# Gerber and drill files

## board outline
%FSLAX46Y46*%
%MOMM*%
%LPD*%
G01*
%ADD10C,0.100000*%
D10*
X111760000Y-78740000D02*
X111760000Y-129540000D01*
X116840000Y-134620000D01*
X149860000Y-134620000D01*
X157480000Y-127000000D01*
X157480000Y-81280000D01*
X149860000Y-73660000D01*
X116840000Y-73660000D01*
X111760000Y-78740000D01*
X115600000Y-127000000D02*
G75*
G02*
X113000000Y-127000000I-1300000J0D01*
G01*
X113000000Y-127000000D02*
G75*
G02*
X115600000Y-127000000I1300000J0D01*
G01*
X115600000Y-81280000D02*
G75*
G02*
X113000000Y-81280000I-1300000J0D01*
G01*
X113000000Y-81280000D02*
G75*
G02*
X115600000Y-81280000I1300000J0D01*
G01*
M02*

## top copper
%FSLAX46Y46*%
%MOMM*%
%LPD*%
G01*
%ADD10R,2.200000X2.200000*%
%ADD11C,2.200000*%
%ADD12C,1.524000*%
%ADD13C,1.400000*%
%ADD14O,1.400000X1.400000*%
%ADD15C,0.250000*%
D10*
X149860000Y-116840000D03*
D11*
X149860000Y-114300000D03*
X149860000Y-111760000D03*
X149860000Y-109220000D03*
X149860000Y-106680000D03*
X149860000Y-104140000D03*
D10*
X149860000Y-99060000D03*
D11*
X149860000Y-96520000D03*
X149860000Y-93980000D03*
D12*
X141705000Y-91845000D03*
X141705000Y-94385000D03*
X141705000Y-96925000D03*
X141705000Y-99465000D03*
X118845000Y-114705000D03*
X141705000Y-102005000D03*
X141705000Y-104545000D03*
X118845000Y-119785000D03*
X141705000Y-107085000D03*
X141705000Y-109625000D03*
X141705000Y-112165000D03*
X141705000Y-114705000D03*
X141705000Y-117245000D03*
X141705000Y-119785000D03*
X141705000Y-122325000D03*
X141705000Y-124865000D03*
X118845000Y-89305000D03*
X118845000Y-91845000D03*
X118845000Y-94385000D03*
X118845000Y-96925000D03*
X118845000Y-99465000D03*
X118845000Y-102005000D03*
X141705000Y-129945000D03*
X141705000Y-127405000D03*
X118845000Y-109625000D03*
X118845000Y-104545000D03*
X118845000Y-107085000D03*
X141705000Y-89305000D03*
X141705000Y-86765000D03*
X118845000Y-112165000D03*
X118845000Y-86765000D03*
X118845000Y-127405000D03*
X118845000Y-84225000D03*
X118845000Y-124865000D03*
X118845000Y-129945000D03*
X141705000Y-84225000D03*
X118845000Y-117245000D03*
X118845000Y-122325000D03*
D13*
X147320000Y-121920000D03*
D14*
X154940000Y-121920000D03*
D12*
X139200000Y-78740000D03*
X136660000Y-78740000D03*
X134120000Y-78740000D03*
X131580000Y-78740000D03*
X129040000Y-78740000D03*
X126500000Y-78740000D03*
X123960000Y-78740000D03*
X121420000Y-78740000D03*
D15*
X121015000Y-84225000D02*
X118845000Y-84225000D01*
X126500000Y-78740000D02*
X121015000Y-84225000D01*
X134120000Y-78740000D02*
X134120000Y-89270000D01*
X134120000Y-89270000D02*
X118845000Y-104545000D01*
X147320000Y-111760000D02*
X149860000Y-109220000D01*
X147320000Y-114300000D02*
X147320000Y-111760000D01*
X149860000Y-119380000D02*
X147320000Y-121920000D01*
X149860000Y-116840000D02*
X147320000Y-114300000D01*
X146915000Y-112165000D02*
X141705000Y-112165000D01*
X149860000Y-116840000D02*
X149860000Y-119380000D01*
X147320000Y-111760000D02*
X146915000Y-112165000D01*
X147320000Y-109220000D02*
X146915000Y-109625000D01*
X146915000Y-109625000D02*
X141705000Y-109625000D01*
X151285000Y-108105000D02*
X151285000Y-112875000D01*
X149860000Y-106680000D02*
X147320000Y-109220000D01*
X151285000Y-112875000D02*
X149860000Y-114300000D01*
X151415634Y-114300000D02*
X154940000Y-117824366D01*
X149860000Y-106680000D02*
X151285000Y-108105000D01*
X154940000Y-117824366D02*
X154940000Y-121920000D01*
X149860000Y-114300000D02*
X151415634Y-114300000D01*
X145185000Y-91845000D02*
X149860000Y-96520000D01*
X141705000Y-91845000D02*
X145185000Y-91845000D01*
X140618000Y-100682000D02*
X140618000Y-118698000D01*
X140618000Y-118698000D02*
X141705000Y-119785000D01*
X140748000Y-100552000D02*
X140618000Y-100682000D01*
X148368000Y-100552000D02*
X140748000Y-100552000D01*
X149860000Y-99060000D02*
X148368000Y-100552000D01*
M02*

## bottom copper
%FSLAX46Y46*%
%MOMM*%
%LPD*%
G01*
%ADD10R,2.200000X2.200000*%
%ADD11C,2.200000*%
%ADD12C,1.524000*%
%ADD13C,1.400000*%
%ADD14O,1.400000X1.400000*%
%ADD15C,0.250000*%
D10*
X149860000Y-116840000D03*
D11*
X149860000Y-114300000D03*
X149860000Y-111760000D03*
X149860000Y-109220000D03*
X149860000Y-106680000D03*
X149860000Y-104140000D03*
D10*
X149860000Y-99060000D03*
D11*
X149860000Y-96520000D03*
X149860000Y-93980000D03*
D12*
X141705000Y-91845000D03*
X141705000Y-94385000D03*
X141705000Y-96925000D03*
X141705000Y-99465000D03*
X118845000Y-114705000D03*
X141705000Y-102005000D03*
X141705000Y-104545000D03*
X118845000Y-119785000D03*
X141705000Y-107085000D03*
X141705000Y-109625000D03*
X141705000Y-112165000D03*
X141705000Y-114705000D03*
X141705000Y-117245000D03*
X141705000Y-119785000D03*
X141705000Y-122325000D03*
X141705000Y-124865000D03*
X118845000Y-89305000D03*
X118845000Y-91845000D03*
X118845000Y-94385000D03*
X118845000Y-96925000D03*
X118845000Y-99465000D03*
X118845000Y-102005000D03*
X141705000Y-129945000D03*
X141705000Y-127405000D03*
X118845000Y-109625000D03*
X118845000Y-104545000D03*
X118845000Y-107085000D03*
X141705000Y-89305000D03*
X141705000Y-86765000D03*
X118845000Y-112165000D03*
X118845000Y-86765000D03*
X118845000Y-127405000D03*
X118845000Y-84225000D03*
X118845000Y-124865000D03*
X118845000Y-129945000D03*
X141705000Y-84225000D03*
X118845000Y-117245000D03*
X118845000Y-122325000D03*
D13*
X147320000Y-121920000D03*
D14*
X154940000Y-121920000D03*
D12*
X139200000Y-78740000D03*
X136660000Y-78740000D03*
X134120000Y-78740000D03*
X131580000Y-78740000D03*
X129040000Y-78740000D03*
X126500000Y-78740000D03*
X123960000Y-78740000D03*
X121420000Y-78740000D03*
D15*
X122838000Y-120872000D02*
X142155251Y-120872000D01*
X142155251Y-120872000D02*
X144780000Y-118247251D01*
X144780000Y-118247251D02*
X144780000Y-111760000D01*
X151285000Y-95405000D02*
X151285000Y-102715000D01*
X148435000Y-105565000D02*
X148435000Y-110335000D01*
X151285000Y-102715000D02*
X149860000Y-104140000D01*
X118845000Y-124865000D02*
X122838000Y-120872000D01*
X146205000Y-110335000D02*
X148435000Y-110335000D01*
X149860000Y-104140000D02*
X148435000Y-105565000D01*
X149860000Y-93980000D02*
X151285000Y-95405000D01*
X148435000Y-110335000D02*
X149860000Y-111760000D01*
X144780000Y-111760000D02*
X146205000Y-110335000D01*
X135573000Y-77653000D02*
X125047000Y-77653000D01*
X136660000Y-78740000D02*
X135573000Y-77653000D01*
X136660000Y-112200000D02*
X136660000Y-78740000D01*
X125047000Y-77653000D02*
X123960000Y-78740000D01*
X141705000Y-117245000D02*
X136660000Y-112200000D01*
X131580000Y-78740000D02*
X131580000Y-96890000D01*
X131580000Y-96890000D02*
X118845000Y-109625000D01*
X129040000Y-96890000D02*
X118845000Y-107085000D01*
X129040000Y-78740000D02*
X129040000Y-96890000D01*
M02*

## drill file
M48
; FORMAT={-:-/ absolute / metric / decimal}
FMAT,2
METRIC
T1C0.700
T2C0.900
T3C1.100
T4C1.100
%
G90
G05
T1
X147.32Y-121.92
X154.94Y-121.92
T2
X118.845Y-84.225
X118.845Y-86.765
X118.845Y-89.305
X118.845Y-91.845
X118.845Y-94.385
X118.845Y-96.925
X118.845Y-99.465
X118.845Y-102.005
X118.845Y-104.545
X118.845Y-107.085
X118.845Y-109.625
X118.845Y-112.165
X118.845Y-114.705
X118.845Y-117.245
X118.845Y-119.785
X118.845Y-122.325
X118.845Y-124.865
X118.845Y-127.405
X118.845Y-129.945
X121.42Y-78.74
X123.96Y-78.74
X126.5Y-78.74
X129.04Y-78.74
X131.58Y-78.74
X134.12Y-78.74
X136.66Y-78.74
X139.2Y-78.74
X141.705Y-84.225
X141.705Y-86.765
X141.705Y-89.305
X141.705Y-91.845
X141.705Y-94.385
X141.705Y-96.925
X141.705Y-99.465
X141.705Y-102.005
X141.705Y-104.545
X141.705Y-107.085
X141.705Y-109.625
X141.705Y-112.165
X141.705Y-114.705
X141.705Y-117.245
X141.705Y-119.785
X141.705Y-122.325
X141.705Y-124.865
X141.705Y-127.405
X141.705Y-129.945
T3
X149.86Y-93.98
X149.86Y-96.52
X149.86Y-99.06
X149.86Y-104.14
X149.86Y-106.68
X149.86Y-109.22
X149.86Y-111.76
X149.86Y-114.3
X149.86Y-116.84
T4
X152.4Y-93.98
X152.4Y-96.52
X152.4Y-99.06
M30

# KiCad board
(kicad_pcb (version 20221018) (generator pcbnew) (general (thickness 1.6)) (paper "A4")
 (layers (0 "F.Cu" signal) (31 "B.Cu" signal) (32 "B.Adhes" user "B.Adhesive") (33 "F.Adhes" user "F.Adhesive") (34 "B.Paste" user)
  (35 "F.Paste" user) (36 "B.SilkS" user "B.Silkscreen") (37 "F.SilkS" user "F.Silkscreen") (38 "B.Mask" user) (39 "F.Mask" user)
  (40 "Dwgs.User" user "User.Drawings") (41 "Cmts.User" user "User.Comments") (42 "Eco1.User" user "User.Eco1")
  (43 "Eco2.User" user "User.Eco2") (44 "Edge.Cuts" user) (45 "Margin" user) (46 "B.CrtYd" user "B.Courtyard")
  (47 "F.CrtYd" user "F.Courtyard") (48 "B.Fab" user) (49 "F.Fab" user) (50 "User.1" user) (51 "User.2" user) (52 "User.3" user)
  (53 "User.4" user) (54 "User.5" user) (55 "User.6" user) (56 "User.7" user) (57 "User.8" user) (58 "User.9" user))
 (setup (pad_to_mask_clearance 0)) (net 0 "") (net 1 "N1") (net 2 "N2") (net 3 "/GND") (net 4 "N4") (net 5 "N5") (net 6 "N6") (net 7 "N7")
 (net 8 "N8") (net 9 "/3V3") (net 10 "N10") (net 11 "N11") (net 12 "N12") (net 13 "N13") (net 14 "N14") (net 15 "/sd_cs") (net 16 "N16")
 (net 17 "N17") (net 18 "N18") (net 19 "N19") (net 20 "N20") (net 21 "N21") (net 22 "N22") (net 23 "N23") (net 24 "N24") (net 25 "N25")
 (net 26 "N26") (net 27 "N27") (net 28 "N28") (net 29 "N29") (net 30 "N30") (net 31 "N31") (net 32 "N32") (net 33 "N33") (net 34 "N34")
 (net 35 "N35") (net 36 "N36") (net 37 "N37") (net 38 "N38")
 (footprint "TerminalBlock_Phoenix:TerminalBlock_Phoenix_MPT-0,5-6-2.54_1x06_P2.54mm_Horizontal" (layer "F.Cu") (at 149.86 116.84 90)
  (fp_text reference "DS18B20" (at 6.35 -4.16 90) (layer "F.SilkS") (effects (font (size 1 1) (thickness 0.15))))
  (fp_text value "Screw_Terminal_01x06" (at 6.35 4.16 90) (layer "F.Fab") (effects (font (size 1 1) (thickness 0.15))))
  (pad "1" thru_hole rect (at 0 0 90) (size 2.2 2.2) (drill 1.1) (layers "*.Cu" "*.Mask") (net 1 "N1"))
  (pad "2" thru_hole circle (at 2.54 0 90) (size 2.2 2.2) (drill 1.1) (layers "*.Cu" "*.Mask") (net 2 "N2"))
  (pad "3" thru_hole circle (at 5.08 0 90) (size 2.2 2.2) (drill 1.1) (layers "*.Cu" "*.Mask") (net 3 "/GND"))
  (pad "4" thru_hole circle (at 7.62 0 90) (size 2.2 2.2) (drill 1.1) (layers "*.Cu" "*.Mask") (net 1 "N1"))
  (pad "5" thru_hole circle (at 10.16 0 90) (size 2.2 2.2) (drill 1.1) (layers "*.Cu" "*.Mask") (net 2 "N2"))
  (pad "6" thru_hole circle (at 12.7 0 90) (size 2.2 2.2) (drill 1.1) (layers "*.Cu" "*.Mask") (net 3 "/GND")))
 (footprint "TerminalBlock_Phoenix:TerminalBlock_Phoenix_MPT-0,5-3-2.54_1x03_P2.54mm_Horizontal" (layer "F.Cu") (at 149.86 99.06 90)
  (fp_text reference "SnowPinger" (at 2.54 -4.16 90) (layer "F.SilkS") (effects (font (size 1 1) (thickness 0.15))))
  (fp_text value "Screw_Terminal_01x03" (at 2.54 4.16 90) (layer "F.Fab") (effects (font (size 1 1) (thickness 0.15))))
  (pad "" np_thru_hole circle (at 0 2.54 90) (size 1.1 1.1) (drill 1.1) (layers "*.Cu" "*.Mask"))
  (pad "" np_thru_hole circle (at 2.54 2.54 90) (size 1.1 1.1) (drill 1.1) (layers "*.Cu" "*.Mask"))
  (pad "" np_thru_hole circle (at 5.08 2.54 90) (size 1.1 1.1) (drill 1.1) (layers "*.Cu" "*.Mask"))
  (pad "1" thru_hole rect (at 0 0 90) (size 2.2 2.2) (drill 1.1) (layers "*.Cu" "*.Mask") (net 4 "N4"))
  (pad "2" thru_hole circle (at 2.54 0 90) (size 2.2 2.2) (drill 1.1) (layers "*.Cu" "*.Mask") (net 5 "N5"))
  (pad "3" thru_hole circle (at 5.08 0 90) (size 2.2 2.2) (drill 1.1) (layers "*.Cu" "*.Mask") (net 3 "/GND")))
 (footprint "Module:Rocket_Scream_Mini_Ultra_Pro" (layer "F.Cu") (at 131.545 107.085)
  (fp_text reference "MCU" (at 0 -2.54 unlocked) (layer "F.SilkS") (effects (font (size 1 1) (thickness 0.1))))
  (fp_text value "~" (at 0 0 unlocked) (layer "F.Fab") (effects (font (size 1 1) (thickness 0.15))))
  (pad "0" thru_hole circle (at 10.16 -15.24) (size 1.524 1.524) (drill 0.9) (layers "*.Cu" "*.Mask") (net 5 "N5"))
  (pad "1" thru_hole circle (at 10.16 -12.7) (size 1.524 1.524) (drill 0.9) (layers "*.Cu" "*.Mask") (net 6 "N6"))
  (pad "2" thru_hole circle (at 10.16 -10.16) (size 1.524 1.524) (drill 0.9) (layers "*.Cu" "*.Mask") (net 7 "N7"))
  (pad "3" thru_hole circle (at 10.16 -7.62) (size 1.524 1.524) (drill 0.9) (layers "*.Cu" "*.Mask") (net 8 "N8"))
  (pad "3V3" thru_hole circle (at -12.7 7.62) (size 1.524 1.524) (drill 0.9) (layers "*.Cu" "*.Mask") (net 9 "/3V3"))
  (pad "4" thru_hole circle (at 10.16 -5.08) (size 1.524 1.524) (drill 0.9) (layers "*.Cu" "*.Mask") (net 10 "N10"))
  (pad "5" thru_hole circle (at 10.16 -2.54) (size 1.524 1.524) (drill 0.9) (layers "*.Cu" "*.Mask") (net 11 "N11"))
  (pad "5V" thru_hole circle (at -12.7 12.7) (size 1.524 1.524) (drill 0.9) (layers "*.Cu" "*.Mask") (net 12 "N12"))
  (pad "6" thru_hole circle (at 10.16 0) (size 1.524 1.524) (drill 0.9) (layers "*.Cu" "*.Mask") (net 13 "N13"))
  (pad "7" thru_hole circle (at 10.16 2.54) (size 1.524 1.524) (drill 0.9) (layers "*.Cu" "*.Mask") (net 2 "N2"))
  (pad "8" thru_hole circle (at 10.16 5.08) (size 1.524 1.524) (drill 0.9) (layers "*.Cu" "*.Mask") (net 1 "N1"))
  (pad "9" thru_hole circle (at 10.16 7.62) (size 1.524 1.524) (drill 0.9) (layers "*.Cu" "*.Mask") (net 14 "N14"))
  (pad "10" thru_hole circle (at 10.16 10.16) (size 1.524 1.524) (drill 0.9) (layers "*.Cu" "*.Mask") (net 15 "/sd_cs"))
  (pad "11" thru_hole circle (at 10.16 12.7) (size 1.524 1.524) (drill 0.9) (layers "*.Cu" "*.Mask") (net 4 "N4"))
  (pad "12" thru_hole circle (at 10.16 15.24) (size 1.524 1.524) (drill 0.9) (layers "*.Cu" "*.Mask") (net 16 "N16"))
  (pad "13" thru_hole circle (at 10.16 17.78) (size 1.524 1.524) (drill 0.9) (layers "*.Cu" "*.Mask") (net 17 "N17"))
  (pad "14" thru_hole circle (at -12.7 -17.78) (size 1.524 1.524) (drill 0.9) (layers "*.Cu" "*.Mask") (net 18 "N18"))
  (pad "15" thru_hole circle (at -12.7 -15.24) (size 1.524 1.524) (drill 0.9) (layers "*.Cu" "*.Mask") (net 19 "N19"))
  (pad "16" thru_hole circle (at -12.7 -12.7) (size 1.524 1.524) (drill 0.9) (layers "*.Cu" "*.Mask") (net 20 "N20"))
  (pad "17" thru_hole circle (at -12.7 -10.16) (size 1.524 1.524) (drill 0.9) (layers "*.Cu" "*.Mask") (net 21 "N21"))
  (pad "18" thru_hole circle (at -12.7 -7.62) (size 1.524 1.524) (drill 0.9) (layers "*.Cu" "*.Mask") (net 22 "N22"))
  (pad "19" thru_hole circle (at -12.7 -5.08) (size 1.524 1.524) (drill 0.9) (layers "*.Cu" "*.Mask") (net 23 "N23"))
  (pad "20" thru_hole circle (at 10.16 22.86) (size 1.524 1.524) (drill 0.9) (layers "*.Cu" "*.Mask") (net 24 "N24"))
  (pad "21" thru_hole circle (at 10.16 20.32) (size 1.524 1.524) (drill 0.9) (layers "*.Cu" "*.Mask") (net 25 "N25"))
  (pad "22" thru_hole circle (at -12.7 2.54) (size 1.524 1.524) (drill 0.9) (layers "*.Cu" "*.Mask") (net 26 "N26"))
  (pad "23" thru_hole circle (at -12.7 -2.54) (size 1.524 1.524) (drill 0.9) (layers "*.Cu" "*.Mask") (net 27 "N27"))
  (pad "24" thru_hole circle (at -12.7 0) (size 1.524 1.524) (drill 0.9) (layers "*.Cu" "*.Mask") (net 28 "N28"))
  (pad "30" thru_hole circle (at 10.16 -17.78) (size 1.524 1.524) (drill 0.9) (layers "*.Cu" "*.Mask") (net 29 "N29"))
  (pad "31" thru_hole circle (at 10.16 -20.32) (size 1.524 1.524) (drill 0.9) (layers "*.Cu" "*.Mask") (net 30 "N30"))
  (pad "38" thru_hole circle (at -12.7 5.08) (size 1.524 1.524) (drill 0.9) (layers "*.Cu" "*.Mask") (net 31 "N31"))
  (pad "AREF" thru_hole circle (at -12.7 -20.32) (size 1.524 1.524) (drill 0.9) (layers "*.Cu" "*.Mask") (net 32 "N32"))
  (pad "BAT" thru_hole circle (at -12.7 20.32) (size 1.524 1.524) (drill 0.9) (layers "*.Cu" "*.Mask") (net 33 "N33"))
  (pad "GND" thru_hole circle (at -12.7 -22.86) (size 1.524 1.524) (drill 0.9) (layers "*.Cu" "*.Mask") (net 3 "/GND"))
  (pad "GND" thru_hole circle (at -12.7 17.78) (size 1.524 1.524) (drill 0.9) (layers "*.Cu" "*.Mask") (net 3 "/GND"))
  (pad "GND" thru_hole circle (at -12.7 22.86) (size 1.524 1.524) (drill 0.9) (layers "*.Cu" "*.Mask") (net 3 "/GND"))
  (pad "RST" thru_hole circle (at 10.16 -22.86) (size 1.524 1.524) (drill 0.9) (layers "*.Cu" "*.Mask") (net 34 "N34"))
  (pad "VBUS" thru_hole circle (at -12.7 10.16) (size 1.524 1.524) (drill 0.9) (layers "*.Cu" "*.Mask") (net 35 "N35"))
  (pad "VIN" thru_hole circle (at -12.7 15.24) (size 1.524 1.524) (drill 0.9) (layers "*.Cu" "*.Mask") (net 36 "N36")))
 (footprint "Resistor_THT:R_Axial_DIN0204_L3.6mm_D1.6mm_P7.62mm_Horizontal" (layer "F.Cu") (at 147.32 121.92)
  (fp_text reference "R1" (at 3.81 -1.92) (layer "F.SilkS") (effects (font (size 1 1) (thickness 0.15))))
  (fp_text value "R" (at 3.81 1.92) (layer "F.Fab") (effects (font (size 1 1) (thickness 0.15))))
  (pad "1" thru_hole circle (at 0 0) (size 1.4 1.4) (drill 0.7) (layers "*.Cu" "*.Mask") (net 1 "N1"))
  (pad "2" thru_hole oval (at 7.62 0) (size 1.4 1.4) (drill 0.7) (layers "*.Cu" "*.Mask") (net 2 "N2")))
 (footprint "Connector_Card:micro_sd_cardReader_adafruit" (layer "B.Cu") (at 129.54 91.44 90)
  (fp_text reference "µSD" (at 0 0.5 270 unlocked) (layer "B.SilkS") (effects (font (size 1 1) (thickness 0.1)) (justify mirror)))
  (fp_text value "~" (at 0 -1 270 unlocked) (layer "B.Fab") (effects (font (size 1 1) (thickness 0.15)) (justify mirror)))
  (pad "1" thru_hole circle (at 12.7 9.66 90) (size 1.524 1.524) (drill 0.9) (layers "*.Cu" "*.Mask") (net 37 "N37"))
  (pad "2" thru_hole circle (at 12.7 7.12 90) (size 1.524 1.524) (drill 0.9) (layers "*.Cu" "*.Mask") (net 15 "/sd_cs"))
  (pad "3" thru_hole circle (at 12.7 4.58 90) (size 1.524 1.524) (drill 0.9) (layers "*.Cu" "*.Mask") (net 27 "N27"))
  (pad "4" thru_hole circle (at 12.7 2.04 90) (size 1.524 1.524) (drill 0.9) (layers "*.Cu" "*.Mask") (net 26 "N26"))
  (pad "5" thru_hole circle (at 12.7 -0.5 90) (size 1.524 1.524) (drill 0.9) (layers "*.Cu" "*.Mask") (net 28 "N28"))
  (pad "6" thru_hole circle (at 12.7 -3.04 90) (size 1.524 1.524) (drill 0.9) (layers "*.Cu" "*.Mask") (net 3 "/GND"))
  (pad "7" thru_hole circle (at 12.7 -5.58 90) (size 1.524 1.524) (drill 0.9) (layers "*.Cu" "*.Mask") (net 15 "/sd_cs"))
  (pad "8" thru_hole circle (at 12.7 -8.12 90) (size 1.524 1.524) (drill 0.9) (layers "*.Cu" "*.Mask") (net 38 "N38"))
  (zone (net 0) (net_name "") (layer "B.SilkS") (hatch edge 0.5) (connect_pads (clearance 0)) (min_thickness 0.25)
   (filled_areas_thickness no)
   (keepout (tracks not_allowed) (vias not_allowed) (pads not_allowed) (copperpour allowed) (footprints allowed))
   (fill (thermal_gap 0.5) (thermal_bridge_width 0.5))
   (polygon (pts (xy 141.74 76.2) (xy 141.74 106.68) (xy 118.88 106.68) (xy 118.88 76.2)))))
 (gr_poly
  (pts (xy 111.76 78.74) (xy 111.76 129.54) (xy 116.84 134.62) (xy 149.86 134.62) (xy 157.48 127) (xy 157.48 81.28) (xy 149.86 73.66)
   (xy 116.84 73.66))
  (stroke (width 0.1) (type solid)) (fill none) (layer "Edge.Cuts"))
 (gr_circle (center 114.3 127) (end 115.6 127) (stroke (width 0.1) (type default)) (fill none) (layer "Edge.Cuts"))
 (gr_circle (center 114.3 81.28) (end 115.6 81.28) (stroke (width 0.1) (type default)) (fill none) (layer "Edge.Cuts"))
 (segment (start 121.015 84.225) (end 118.845 84.225) (width 0.25) (layer "F.Cu") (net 3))
 (segment (start 126.5 78.74) (end 121.015 84.225) (width 0.25) (layer "F.Cu") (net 3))
 (segment (start 122.838 120.872) (end 142.155251 120.872) (width 0.25) (layer "B.Cu") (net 3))
 (segment (start 142.155251 120.872) (end 144.78 118.247251) (width 0.25) (layer "B.Cu") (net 3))
 (segment (start 144.78 118.247251) (end 144.78 111.76) (width 0.25) (layer "B.Cu") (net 3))
 (segment (start 151.285 95.405) (end 151.285 102.715) (width 0.25) (layer "B.Cu") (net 3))
 (segment (start 148.435 105.565) (end 148.435 110.335) (width 0.25) (layer "B.Cu") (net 3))
 (segment (start 151.285 102.715) (end 149.86 104.14) (width 0.25) (layer "B.Cu") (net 3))
 (segment (start 118.845 124.865) (end 122.838 120.872) (width 0.25) (layer "B.Cu") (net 3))
 (segment (start 146.205 110.335) (end 148.435 110.335) (width 0.25) (layer "B.Cu") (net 3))
 (segment (start 149.86 104.14) (end 148.435 105.565) (width 0.25) (layer "B.Cu") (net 3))
 (segment (start 149.86 93.98) (end 151.285 95.405) (width 0.25) (layer "B.Cu") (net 3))
 (segment (start 148.435 110.335) (end 149.86 111.76) (width 0.25) (layer "B.Cu") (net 3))
 (segment (start 144.78 111.76) (end 146.205 110.335) (width 0.25) (layer "B.Cu") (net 3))
 (segment (start 135.573 77.653) (end 125.047 77.653) (width 0.25) (layer "B.Cu") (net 15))
 (segment (start 136.66 78.74) (end 135.573 77.653) (width 0.25) (layer "B.Cu") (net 15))
 (segment (start 136.66 112.2) (end 136.66 78.74) (width 0.25) (layer "B.Cu") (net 15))
 (segment (start 125.047 77.653) (end 123.96 78.74) (width 0.25) (layer "B.Cu") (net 15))
 (segment (start 141.705 117.245) (end 136.66 112.2) (width 0.25) (layer "B.Cu") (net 15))
 (segment (start 131.58 78.74) (end 131.58 96.89) (width 0.25) (layer "B.Cu") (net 26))
 (segment (start 131.58 96.89) (end 118.845 109.625) (width 0.25) (layer "B.Cu") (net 26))
 (segment (start 134.12 78.74) (end 134.12 89.27) (width 0.25) (layer "F.Cu") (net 27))
 (segment (start 134.12 89.27) (end 118.845 104.545) (width 0.25) (layer "F.Cu") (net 27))
 (segment (start 129.04 96.89) (end 118.845 107.085) (width 0.25) (layer "B.Cu") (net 28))
 (segment (start 129.04 78.74) (end 129.04 96.89) (width 0.25) (layer "B.Cu") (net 28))
 (segment (start 147.32 111.76) (end 149.86 109.22) (width 0.25) (layer "F.Cu") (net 1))
 (segment (start 147.32 114.3) (end 147.32 111.76) (width 0.25) (layer "F.Cu") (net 1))
 (segment (start 149.86 119.38) (end 147.32 121.92) (width 0.25) (layer "F.Cu") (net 1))
 (segment (start 149.86 116.84) (end 147.32 114.3) (width 0.25) (layer "F.Cu") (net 1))
 (segment (start 146.915 112.165) (end 141.705 112.165) (width 0.25) (layer "F.Cu") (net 1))
 (segment (start 149.86 116.84) (end 149.86 119.38) (width 0.25) (layer "F.Cu") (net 1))
 (segment (start 147.32 111.76) (end 146.915 112.165) (width 0.25) (layer "F.Cu") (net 1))
 (segment (start 147.32 109.22) (end 146.915 109.625) (width 0.25) (layer "F.Cu") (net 2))
 (segment (start 146.915 109.625) (end 141.705 109.625) (width 0.25) (layer "F.Cu") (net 2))
 (segment (start 151.285 108.105) (end 151.285 112.875) (width 0.25) (layer "F.Cu") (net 2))
 (segment (start 149.86 106.68) (end 147.32 109.22) (width 0.25) (layer "F.Cu") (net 2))
 (segment (start 151.285 112.875) (end 149.86 114.3) (width 0.25) (layer "F.Cu") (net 2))
 (segment (start 151.415634 114.3) (end 154.94 117.824366) (width 0.25) (layer "F.Cu") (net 2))
 (segment (start 149.86 106.68) (end 151.285 108.105) (width 0.25) (layer "F.Cu") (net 2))
 (segment (start 154.94 117.824366) (end 154.94 121.92) (width 0.25) (layer "F.Cu") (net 2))
 (segment (start 149.86 114.3) (end 151.415634 114.3) (width 0.25) (layer "F.Cu") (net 2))
 (segment (start 145.185 91.845) (end 149.86 96.52) (width 0.25) (layer "F.Cu") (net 5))
 (segment (start 141.705 91.845) (end 145.185 91.845) (width 0.25) (layer "F.Cu") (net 5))
 (segment (start 140.618 100.682) (end 140.618 118.698) (width 0.25) (layer "F.Cu") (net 4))
 (segment (start 140.618 118.698) (end 141.705 119.785) (width 0.25) (layer "F.Cu") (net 4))
 (segment (start 140.748 100.552) (end 140.618 100.682) (width 0.25) (layer "F.Cu") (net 4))
 (segment (start 148.368 100.552) (end 140.748 100.552) (width 0.25) (layer "F.Cu") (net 4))
 (segment (start 149.86 99.06) (end 148.368 100.552) (width 0.25) (layer "F.Cu") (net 4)))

